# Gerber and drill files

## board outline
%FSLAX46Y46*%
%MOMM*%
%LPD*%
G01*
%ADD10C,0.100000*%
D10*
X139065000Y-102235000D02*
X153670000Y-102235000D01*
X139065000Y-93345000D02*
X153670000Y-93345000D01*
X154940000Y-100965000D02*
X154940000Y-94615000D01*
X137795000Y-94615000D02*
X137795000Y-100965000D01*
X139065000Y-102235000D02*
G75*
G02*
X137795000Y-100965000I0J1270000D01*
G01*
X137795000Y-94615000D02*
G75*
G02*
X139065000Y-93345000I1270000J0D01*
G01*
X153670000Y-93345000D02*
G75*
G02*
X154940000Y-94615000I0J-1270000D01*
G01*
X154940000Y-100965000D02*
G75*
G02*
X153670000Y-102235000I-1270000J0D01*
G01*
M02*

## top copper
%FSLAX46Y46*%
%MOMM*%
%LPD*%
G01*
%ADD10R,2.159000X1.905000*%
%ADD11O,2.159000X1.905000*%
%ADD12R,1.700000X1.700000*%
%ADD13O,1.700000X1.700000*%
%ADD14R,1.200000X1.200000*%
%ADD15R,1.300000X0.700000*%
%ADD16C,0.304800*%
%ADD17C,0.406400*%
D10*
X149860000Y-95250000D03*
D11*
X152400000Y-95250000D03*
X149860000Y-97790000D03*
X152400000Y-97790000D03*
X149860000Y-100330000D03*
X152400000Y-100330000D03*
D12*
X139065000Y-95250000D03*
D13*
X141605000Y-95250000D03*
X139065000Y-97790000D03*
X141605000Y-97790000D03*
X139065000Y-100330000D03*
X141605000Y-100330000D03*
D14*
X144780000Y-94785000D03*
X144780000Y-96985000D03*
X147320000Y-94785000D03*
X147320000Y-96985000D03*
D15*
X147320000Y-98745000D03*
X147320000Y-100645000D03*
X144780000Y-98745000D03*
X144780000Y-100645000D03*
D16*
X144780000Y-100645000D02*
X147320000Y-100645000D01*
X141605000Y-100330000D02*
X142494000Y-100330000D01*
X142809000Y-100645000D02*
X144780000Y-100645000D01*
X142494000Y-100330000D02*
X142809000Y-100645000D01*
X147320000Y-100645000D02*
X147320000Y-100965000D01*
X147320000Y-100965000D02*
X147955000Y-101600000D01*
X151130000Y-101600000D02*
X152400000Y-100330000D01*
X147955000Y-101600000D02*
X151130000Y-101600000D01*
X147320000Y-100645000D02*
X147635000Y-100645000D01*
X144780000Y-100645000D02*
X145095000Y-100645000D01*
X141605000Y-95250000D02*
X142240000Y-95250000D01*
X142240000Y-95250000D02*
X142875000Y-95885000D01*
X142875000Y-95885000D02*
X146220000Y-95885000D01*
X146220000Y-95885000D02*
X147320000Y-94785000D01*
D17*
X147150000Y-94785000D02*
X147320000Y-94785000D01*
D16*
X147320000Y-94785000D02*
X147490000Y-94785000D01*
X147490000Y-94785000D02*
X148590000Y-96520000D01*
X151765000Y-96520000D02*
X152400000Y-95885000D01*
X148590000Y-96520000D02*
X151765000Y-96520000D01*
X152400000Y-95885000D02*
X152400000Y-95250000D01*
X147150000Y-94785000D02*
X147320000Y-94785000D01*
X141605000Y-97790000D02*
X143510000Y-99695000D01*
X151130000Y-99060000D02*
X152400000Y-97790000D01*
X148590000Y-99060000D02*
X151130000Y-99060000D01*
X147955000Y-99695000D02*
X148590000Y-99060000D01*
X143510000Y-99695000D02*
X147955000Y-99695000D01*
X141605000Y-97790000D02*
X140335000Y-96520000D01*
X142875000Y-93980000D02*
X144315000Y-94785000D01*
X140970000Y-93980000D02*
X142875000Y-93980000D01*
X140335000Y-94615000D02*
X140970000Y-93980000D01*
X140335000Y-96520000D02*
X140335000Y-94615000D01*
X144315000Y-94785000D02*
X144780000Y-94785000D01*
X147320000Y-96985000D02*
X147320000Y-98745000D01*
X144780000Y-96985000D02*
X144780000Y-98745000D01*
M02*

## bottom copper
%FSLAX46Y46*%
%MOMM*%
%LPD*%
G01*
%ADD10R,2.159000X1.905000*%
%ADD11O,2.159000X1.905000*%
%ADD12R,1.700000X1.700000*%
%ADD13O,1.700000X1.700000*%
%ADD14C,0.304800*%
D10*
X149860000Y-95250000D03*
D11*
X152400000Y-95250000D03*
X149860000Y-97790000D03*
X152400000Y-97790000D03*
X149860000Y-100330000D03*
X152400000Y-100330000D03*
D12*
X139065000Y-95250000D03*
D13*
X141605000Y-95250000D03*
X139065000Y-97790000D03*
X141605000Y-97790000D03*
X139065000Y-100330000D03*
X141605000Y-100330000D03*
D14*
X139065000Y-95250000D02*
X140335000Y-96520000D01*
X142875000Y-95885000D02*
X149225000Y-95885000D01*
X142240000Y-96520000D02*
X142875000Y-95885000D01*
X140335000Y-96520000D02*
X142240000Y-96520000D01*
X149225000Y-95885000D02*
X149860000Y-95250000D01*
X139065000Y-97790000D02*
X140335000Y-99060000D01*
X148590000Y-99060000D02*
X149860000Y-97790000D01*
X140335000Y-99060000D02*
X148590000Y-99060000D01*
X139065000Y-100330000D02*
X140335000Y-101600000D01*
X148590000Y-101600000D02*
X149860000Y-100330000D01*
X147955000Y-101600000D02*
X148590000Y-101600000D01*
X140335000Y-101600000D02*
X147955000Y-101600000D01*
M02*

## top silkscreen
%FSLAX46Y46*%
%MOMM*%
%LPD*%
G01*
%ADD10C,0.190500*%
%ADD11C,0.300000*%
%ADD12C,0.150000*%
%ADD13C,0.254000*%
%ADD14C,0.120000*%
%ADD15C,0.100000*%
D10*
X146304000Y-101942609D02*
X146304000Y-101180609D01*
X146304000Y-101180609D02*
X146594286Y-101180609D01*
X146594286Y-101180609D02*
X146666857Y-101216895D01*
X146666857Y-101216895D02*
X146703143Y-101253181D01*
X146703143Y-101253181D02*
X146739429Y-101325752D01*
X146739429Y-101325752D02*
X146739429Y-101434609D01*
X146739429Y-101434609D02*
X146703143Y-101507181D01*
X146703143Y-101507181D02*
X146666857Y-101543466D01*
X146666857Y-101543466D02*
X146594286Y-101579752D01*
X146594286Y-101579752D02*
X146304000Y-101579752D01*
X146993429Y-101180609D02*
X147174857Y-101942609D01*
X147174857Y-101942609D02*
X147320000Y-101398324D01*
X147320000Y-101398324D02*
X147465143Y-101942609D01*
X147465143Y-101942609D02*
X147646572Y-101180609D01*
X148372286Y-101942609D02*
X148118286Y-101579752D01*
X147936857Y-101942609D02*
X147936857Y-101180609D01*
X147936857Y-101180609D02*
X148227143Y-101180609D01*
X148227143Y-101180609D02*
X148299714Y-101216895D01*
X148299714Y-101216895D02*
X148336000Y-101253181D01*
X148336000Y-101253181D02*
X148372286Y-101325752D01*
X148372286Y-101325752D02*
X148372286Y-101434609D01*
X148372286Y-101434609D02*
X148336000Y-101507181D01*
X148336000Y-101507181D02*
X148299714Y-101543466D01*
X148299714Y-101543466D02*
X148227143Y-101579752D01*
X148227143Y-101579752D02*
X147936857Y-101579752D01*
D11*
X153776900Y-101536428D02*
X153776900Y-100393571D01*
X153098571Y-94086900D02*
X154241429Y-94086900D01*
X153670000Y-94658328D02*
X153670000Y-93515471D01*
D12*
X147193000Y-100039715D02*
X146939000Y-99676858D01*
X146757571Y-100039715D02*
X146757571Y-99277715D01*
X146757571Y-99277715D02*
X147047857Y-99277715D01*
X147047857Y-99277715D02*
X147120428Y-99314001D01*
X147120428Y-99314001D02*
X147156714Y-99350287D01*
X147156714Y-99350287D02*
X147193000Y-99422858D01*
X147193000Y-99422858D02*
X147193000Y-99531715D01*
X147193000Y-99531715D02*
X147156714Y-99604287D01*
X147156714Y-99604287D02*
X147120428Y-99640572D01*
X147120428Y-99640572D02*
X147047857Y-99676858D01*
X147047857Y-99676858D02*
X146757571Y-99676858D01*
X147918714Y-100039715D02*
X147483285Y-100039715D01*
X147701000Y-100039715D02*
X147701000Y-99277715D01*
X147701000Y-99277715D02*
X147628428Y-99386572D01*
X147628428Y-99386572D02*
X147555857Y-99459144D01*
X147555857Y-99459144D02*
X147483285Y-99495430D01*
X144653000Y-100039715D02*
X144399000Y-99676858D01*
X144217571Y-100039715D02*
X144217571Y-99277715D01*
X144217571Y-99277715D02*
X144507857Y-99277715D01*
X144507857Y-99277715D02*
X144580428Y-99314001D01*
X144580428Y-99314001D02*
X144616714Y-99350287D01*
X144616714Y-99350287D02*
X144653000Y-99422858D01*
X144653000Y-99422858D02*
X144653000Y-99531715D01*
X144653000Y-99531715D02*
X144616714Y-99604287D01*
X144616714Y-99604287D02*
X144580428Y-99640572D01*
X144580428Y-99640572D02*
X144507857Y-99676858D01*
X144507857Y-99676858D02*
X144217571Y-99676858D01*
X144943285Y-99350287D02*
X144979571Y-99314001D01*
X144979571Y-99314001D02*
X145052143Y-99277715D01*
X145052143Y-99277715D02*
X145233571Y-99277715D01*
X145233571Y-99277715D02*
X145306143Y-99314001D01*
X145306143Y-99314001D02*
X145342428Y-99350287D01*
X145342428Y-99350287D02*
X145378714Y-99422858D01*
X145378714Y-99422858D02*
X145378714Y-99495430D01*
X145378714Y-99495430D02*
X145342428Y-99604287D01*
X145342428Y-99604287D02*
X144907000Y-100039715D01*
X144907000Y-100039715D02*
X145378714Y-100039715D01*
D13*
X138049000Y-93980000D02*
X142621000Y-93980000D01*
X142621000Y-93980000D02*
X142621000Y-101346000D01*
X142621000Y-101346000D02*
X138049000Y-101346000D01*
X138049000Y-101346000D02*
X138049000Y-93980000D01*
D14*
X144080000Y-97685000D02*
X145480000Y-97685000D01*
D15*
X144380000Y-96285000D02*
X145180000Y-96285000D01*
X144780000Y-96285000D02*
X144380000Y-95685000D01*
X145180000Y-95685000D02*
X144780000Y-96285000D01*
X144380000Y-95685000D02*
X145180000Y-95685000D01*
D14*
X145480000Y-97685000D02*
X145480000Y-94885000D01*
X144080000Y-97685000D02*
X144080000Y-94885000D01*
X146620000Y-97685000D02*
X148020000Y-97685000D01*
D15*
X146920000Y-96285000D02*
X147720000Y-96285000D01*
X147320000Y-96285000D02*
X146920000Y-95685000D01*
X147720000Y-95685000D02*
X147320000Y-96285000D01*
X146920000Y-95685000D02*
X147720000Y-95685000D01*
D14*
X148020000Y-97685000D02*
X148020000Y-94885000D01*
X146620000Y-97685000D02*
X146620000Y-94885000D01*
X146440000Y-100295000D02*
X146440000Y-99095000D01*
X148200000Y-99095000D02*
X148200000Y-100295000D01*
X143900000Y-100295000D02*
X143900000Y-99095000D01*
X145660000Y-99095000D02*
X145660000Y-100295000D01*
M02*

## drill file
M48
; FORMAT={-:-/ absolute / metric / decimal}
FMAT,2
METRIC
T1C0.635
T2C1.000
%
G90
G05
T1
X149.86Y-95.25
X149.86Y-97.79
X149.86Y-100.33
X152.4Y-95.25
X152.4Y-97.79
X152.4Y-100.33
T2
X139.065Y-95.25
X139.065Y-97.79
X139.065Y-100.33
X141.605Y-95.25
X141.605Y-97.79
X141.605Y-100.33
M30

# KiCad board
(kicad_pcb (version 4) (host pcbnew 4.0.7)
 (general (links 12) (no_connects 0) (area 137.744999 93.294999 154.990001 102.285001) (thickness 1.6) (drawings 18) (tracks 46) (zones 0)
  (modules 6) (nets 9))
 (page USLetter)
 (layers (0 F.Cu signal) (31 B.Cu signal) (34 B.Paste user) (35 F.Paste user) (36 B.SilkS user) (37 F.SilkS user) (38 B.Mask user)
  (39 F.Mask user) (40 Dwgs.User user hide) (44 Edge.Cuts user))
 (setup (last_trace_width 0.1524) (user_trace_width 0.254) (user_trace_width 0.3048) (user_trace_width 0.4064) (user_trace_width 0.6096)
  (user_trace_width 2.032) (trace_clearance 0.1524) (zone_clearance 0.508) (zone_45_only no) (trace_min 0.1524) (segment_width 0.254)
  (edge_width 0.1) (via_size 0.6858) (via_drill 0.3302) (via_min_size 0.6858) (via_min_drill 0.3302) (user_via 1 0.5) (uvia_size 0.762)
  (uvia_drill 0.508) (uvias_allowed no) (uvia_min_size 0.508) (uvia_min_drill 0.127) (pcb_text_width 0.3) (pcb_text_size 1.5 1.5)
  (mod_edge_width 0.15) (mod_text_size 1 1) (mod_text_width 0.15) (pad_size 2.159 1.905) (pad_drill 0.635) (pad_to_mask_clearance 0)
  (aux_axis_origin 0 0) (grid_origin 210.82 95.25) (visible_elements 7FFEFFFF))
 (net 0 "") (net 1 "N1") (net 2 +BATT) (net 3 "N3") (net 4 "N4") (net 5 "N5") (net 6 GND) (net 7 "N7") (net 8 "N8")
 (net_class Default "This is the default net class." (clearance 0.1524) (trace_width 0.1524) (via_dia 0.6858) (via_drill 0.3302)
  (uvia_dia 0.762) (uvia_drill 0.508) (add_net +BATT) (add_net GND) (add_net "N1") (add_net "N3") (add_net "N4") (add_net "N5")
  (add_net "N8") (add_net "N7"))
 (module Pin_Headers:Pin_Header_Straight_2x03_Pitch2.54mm (layer F.Cu) (at 149.86 95.25)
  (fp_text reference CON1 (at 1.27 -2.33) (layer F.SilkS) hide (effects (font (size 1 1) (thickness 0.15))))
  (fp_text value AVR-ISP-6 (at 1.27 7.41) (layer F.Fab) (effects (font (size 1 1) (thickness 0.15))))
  (pad 1 thru_hole rect (at 0 0) (size 2.159 1.905) (drill 0.635) (layers *.Cu *.Mask) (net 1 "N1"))
  (pad 2 thru_hole oval (at 2.54 0) (size 2.159 1.905) (drill 0.635) (layers *.Cu *.Mask) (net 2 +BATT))
  (pad 3 thru_hole oval (at 0 2.54) (size 2.159 1.905) (drill 0.635) (layers *.Cu *.Mask) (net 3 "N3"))
  (pad 4 thru_hole oval (at 2.54 2.54) (size 2.159 1.905) (drill 0.635) (layers *.Cu *.Mask) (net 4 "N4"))
  (pad 5 thru_hole oval (at 0 5.08) (size 2.159 1.905) (drill 0.635) (layers *.Cu *.Mask) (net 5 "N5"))
  (pad 6 thru_hole oval (at 2.54 5.08) (size 2.159 1.905) (drill 0.635) (layers *.Cu *.Mask) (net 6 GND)))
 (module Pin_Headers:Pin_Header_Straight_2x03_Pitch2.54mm (layer F.Cu) (at 139.065 95.25)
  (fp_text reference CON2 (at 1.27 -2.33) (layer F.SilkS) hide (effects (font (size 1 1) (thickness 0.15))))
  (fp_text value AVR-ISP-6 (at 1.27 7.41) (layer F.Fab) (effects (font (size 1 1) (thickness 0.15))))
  (fp_line (start -1.016 -1.27) (end 3.556 -1.27) (layer F.SilkS) (width 0.254))
  (fp_line (start 3.556 -1.27) (end 3.556 6.096) (layer F.SilkS) (width 0.254))
  (fp_line (start 3.556 6.096) (end -1.016 6.096) (layer F.SilkS) (width 0.254))
  (fp_line (start -1.016 6.096) (end -1.016 -1.27) (layer F.SilkS) (width 0.254))
  (pad 1 thru_hole rect (at 0 0) (size 1.7 1.7) (drill 1) (layers *.Cu *.Mask) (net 1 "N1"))
  (pad 2 thru_hole oval (at 2.54 0) (size 1.7 1.7) (drill 1) (layers *.Cu *.Mask) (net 2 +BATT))
  (pad 3 thru_hole oval (at 0 2.54) (size 1.7 1.7) (drill 1) (layers *.Cu *.Mask) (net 3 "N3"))
  (pad 4 thru_hole oval (at 2.54 2.54) (size 1.7 1.7) (drill 1) (layers *.Cu *.Mask) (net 4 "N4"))
  (pad 5 thru_hole oval (at 0 5.08) (size 1.7 1.7) (drill 1) (layers *.Cu *.Mask) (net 5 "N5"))
  (pad 6 thru_hole oval (at 2.54 5.08) (size 1.7 1.7) (drill 1) (layers *.Cu *.Mask) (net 6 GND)))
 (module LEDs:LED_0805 (layer F.Cu) (at 144.78 95.885 90)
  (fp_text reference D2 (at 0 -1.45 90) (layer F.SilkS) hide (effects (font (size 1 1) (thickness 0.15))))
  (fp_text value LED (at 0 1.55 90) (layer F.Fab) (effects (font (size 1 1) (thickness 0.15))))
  (fp_line (start -1.8 -0.7) (end -1.8 0.7) (layer F.SilkS) (width 0.12))
  (fp_line (start -0.4 -0.4) (end -0.4 0.4) (layer F.SilkS) (width 0.1))
  (fp_line (start -0.4 0) (end 0.2 -0.4) (layer F.SilkS) (width 0.1))
  (fp_line (start 0.2 0.4) (end -0.4 0) (layer F.SilkS) (width 0.1))
  (fp_line (start 0.2 -0.4) (end 0.2 0.4) (layer F.SilkS) (width 0.1))
  (fp_line (start -1.8 0.7) (end 1 0.7) (layer F.SilkS) (width 0.12))
  (fp_line (start -1.8 -0.7) (end 1 -0.7) (layer F.SilkS) (width 0.12))
  (pad 2 smd rect (at 1.1 0 270) (size 1.2 1.2) (layers F.Cu F.Paste F.Mask) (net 4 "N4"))
  (pad 1 smd rect (at -1.1 0 270) (size 1.2 1.2) (layers F.Cu F.Paste F.Mask) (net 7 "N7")))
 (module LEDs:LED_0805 (layer F.Cu) (at 147.32 95.885 90)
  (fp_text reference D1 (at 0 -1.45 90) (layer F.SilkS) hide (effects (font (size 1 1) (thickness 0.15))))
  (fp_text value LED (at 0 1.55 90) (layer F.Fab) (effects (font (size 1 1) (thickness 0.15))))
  (fp_line (start -1.8 -0.7) (end -1.8 0.7) (layer F.SilkS) (width 0.12))
  (fp_line (start -0.4 -0.4) (end -0.4 0.4) (layer F.SilkS) (width 0.1))
  (fp_line (start -0.4 0) (end 0.2 -0.4) (layer F.SilkS) (width 0.1))
  (fp_line (start 0.2 0.4) (end -0.4 0) (layer F.SilkS) (width 0.1))
  (fp_line (start 0.2 -0.4) (end 0.2 0.4) (layer F.SilkS) (width 0.1))
  (fp_line (start -1.8 0.7) (end 1 0.7) (layer F.SilkS) (width 0.12))
  (fp_line (start -1.8 -0.7) (end 1 -0.7) (layer F.SilkS) (width 0.12))
  (pad 2 smd rect (at 1.1 0 270) (size 1.2 1.2) (layers F.Cu F.Paste F.Mask) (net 2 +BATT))
  (pad 1 smd rect (at -1.1 0 270) (size 1.2 1.2) (layers F.Cu F.Paste F.Mask) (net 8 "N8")))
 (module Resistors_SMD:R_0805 (layer F.Cu) (at 147.32 99.695 270)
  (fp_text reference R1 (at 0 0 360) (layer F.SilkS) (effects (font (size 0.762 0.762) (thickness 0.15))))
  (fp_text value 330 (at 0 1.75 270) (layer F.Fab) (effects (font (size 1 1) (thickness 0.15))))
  (fp_line (start 0.6 0.88) (end -0.6 0.88) (layer F.SilkS) (width 0.12))
  (fp_line (start -0.6 -0.88) (end 0.6 -0.88) (layer F.SilkS) (width 0.12))
  (pad 1 smd rect (at -0.95 0 270) (size 0.7 1.3) (layers F.Cu F.Paste F.Mask) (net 8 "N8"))
  (pad 2 smd rect (at 0.95 0 270) (size 0.7 1.3) (layers F.Cu F.Paste F.Mask) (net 6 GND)))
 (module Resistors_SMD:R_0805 (layer F.Cu) (at 144.78 99.695 270)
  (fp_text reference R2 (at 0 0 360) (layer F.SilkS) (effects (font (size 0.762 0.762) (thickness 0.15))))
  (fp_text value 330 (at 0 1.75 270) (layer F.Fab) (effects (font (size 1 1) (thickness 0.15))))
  (fp_line (start 0.6 0.88) (end -0.6 0.88) (layer F.SilkS) (width 0.12))
  (fp_line (start -0.6 -0.88) (end 0.6 -0.88) (layer F.SilkS) (width 0.12))
  (pad 1 smd rect (at -0.95 0 270) (size 0.7 1.3) (layers F.Cu F.Paste F.Mask) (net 7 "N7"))
  (pad 2 smd rect (at 0.95 0 270) (size 0.7 1.3) (layers F.Cu F.Paste F.Mask) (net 6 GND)))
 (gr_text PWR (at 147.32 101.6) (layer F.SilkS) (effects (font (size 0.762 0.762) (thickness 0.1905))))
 (gr_line (start 139.065 102.235) (end 153.67 102.235) (angle 90) (layer Edge.Cuts) (width 0.1))
 (gr_line (start 139.065 93.345) (end 153.67 93.345) (angle 90) (layer Edge.Cuts) (width 0.1))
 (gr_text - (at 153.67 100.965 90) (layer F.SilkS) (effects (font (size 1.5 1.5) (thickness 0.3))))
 (gr_line (start 154.94 100.965) (end 154.94 94.615) (angle 90) (layer Edge.Cuts) (width 0.1))
 (gr_line (start 137.795 94.615) (end 137.795 100.965) (angle 90) (layer Edge.Cuts) (width 0.1))
 (gr_arc (start 139.065 100.965) (end 139.065 102.235) (angle 90) (layer Edge.Cuts) (width 0.1))
 (gr_arc (start 139.065 94.615) (end 137.795 94.615) (angle 90) (layer Edge.Cuts) (width 0.1))
 (gr_arc (start 153.67 94.615) (end 153.67 93.345) (angle 90) (layer Edge.Cuts) (width 0.1))
 (gr_arc (start 153.67 100.965) (end 154.94 100.965) (angle 90) (layer Edge.Cuts) (width 0.1))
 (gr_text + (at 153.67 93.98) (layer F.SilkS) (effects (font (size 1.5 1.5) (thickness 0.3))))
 (segment (start 144.78 100.645) (end 147.32 100.645) (width 0.3048) (layer F.Cu) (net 6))
 (segment (start 141.605 100.33) (end 142.494 100.33) (width 0.3048) (layer F.Cu) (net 6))
 (segment (start 142.809 100.645) (end 144.78 100.645) (width 0.3048) (layer F.Cu) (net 6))
 (segment (start 142.494 100.33) (end 142.809 100.645) (width 0.3048) (layer F.Cu) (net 6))
 (segment (start 147.32 100.645) (end 147.32 100.965) (width 0.3048) (layer F.Cu) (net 6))
 (segment (start 147.32 100.965) (end 147.955 101.6) (width 0.3048) (layer F.Cu) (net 6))
 (segment (start 151.13 101.6) (end 152.4 100.33) (width 0.3048) (layer F.Cu) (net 6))
 (segment (start 147.955 101.6) (end 151.13 101.6) (width 0.3048) (layer F.Cu) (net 6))
 (segment (start 147.32 100.645) (end 147.635 100.645) (width 0.3048) (layer F.Cu) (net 6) (status 30))
 (segment (start 144.78 100.645) (end 145.095 100.645) (width 0.3048) (layer F.Cu) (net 6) (status 30))
 (segment (start 141.605 95.25) (end 142.24 95.25) (width 0.3048) (layer F.Cu) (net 2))
 (segment (start 142.24 95.25) (end 142.875 95.885) (width 0.3048) (layer F.Cu) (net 2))
 (segment (start 142.875 95.885) (end 146.22 95.885) (width 0.3048) (layer F.Cu) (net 2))
 (segment (start 146.22 95.885) (end 147.32 94.785) (width 0.3048) (layer F.Cu) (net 2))
 (segment (start 147.15 94.785) (end 147.32 94.785) (width 0.4064) (layer F.Cu) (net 2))
 (segment (start 147.32 94.785) (end 147.49 94.785) (width 0.3048) (layer F.Cu) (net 2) (status 30))
 (segment (start 147.49 94.785) (end 148.59 96.52) (width 0.3048) (layer F.Cu) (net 2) (status 10))
 (segment (start 151.765 96.52) (end 152.4 95.885) (width 0.3048) (layer F.Cu) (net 2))
 (segment (start 148.59 96.52) (end 151.765 96.52) (width 0.3048) (layer F.Cu) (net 2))
 (segment (start 152.4 95.885) (end 152.4 95.25) (width 0.3048) (layer F.Cu) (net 2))
 (segment (start 147.15 94.785) (end 147.32 94.785) (width 0.3048) (layer F.Cu) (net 2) (status 30))
 (segment (start 139.065 95.25) (end 140.335 96.52) (width 0.3048) (layer B.Cu) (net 1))
 (segment (start 142.875 95.885) (end 149.225 95.885) (width 0.3048) (layer B.Cu) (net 1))
 (segment (start 142.24 96.52) (end 142.875 95.885) (width 0.3048) (layer B.Cu) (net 1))
 (segment (start 140.335 96.52) (end 142.24 96.52) (width 0.3048) (layer B.Cu) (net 1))
 (segment (start 149.225 95.885) (end 149.86 95.25) (width 0.3048) (layer B.Cu) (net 1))
 (segment (start 139.065 97.79) (end 140.335 99.06) (width 0.3048) (layer B.Cu) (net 3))
 (segment (start 148.59 99.06) (end 149.86 97.79) (width 0.3048) (layer B.Cu) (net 3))
 (segment (start 140.335 99.06) (end 148.59 99.06) (width 0.3048) (layer B.Cu) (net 3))
 (segment (start 141.605 97.79) (end 143.51 99.695) (width 0.3048) (layer F.Cu) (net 4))
 (segment (start 151.13 99.06) (end 152.4 97.79) (width 0.3048) (layer F.Cu) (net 4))
 (segment (start 148.59 99.06) (end 151.13 99.06) (width 0.3048) (layer F.Cu) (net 4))
 (segment (start 147.955 99.695) (end 148.59 99.06) (width 0.3048) (layer F.Cu) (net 4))
 (segment (start 143.51 99.695) (end 147.955 99.695) (width 0.3048) (layer F.Cu) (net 4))
 (segment (start 141.605 97.79) (end 140.335 96.52) (width 0.3048) (layer F.Cu) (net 4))
 (segment (start 142.875 93.98) (end 144.315 94.785) (width 0.3048) (layer F.Cu) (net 4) (status 20))
 (segment (start 140.97 93.98) (end 142.875 93.98) (width 0.3048) (layer F.Cu) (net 4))
 (segment (start 140.335 94.615) (end 140.97 93.98) (width 0.3048) (layer F.Cu) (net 4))
 (segment (start 140.335 96.52) (end 140.335 94.615) (width 0.3048) (layer F.Cu) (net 4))
 (segment (start 144.315 94.785) (end 144.78 94.785) (width 0.3048) (layer F.Cu) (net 4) (status 30))
 (segment (start 139.065 100.33) (end 140.335 101.6) (width 0.3048) (layer B.Cu) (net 5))
 (segment (start 148.59 101.6) (end 149.86 100.33) (width 0.3048) (layer B.Cu) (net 5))
 (segment (start 147.955 101.6) (end 148.59 101.6) (width 0.3048) (layer B.Cu) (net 5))
 (segment (start 140.335 101.6) (end 147.955 101.6) (width 0.3048) (layer B.Cu) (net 5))
 (segment (start 147.32 96.985) (end 147.32 98.745) (width 0.3048) (layer F.Cu) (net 8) (status 20))
 (segment (start 144.78 96.985) (end 144.78 98.745) (width 0.3048) (layer F.Cu) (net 7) (status 10)))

